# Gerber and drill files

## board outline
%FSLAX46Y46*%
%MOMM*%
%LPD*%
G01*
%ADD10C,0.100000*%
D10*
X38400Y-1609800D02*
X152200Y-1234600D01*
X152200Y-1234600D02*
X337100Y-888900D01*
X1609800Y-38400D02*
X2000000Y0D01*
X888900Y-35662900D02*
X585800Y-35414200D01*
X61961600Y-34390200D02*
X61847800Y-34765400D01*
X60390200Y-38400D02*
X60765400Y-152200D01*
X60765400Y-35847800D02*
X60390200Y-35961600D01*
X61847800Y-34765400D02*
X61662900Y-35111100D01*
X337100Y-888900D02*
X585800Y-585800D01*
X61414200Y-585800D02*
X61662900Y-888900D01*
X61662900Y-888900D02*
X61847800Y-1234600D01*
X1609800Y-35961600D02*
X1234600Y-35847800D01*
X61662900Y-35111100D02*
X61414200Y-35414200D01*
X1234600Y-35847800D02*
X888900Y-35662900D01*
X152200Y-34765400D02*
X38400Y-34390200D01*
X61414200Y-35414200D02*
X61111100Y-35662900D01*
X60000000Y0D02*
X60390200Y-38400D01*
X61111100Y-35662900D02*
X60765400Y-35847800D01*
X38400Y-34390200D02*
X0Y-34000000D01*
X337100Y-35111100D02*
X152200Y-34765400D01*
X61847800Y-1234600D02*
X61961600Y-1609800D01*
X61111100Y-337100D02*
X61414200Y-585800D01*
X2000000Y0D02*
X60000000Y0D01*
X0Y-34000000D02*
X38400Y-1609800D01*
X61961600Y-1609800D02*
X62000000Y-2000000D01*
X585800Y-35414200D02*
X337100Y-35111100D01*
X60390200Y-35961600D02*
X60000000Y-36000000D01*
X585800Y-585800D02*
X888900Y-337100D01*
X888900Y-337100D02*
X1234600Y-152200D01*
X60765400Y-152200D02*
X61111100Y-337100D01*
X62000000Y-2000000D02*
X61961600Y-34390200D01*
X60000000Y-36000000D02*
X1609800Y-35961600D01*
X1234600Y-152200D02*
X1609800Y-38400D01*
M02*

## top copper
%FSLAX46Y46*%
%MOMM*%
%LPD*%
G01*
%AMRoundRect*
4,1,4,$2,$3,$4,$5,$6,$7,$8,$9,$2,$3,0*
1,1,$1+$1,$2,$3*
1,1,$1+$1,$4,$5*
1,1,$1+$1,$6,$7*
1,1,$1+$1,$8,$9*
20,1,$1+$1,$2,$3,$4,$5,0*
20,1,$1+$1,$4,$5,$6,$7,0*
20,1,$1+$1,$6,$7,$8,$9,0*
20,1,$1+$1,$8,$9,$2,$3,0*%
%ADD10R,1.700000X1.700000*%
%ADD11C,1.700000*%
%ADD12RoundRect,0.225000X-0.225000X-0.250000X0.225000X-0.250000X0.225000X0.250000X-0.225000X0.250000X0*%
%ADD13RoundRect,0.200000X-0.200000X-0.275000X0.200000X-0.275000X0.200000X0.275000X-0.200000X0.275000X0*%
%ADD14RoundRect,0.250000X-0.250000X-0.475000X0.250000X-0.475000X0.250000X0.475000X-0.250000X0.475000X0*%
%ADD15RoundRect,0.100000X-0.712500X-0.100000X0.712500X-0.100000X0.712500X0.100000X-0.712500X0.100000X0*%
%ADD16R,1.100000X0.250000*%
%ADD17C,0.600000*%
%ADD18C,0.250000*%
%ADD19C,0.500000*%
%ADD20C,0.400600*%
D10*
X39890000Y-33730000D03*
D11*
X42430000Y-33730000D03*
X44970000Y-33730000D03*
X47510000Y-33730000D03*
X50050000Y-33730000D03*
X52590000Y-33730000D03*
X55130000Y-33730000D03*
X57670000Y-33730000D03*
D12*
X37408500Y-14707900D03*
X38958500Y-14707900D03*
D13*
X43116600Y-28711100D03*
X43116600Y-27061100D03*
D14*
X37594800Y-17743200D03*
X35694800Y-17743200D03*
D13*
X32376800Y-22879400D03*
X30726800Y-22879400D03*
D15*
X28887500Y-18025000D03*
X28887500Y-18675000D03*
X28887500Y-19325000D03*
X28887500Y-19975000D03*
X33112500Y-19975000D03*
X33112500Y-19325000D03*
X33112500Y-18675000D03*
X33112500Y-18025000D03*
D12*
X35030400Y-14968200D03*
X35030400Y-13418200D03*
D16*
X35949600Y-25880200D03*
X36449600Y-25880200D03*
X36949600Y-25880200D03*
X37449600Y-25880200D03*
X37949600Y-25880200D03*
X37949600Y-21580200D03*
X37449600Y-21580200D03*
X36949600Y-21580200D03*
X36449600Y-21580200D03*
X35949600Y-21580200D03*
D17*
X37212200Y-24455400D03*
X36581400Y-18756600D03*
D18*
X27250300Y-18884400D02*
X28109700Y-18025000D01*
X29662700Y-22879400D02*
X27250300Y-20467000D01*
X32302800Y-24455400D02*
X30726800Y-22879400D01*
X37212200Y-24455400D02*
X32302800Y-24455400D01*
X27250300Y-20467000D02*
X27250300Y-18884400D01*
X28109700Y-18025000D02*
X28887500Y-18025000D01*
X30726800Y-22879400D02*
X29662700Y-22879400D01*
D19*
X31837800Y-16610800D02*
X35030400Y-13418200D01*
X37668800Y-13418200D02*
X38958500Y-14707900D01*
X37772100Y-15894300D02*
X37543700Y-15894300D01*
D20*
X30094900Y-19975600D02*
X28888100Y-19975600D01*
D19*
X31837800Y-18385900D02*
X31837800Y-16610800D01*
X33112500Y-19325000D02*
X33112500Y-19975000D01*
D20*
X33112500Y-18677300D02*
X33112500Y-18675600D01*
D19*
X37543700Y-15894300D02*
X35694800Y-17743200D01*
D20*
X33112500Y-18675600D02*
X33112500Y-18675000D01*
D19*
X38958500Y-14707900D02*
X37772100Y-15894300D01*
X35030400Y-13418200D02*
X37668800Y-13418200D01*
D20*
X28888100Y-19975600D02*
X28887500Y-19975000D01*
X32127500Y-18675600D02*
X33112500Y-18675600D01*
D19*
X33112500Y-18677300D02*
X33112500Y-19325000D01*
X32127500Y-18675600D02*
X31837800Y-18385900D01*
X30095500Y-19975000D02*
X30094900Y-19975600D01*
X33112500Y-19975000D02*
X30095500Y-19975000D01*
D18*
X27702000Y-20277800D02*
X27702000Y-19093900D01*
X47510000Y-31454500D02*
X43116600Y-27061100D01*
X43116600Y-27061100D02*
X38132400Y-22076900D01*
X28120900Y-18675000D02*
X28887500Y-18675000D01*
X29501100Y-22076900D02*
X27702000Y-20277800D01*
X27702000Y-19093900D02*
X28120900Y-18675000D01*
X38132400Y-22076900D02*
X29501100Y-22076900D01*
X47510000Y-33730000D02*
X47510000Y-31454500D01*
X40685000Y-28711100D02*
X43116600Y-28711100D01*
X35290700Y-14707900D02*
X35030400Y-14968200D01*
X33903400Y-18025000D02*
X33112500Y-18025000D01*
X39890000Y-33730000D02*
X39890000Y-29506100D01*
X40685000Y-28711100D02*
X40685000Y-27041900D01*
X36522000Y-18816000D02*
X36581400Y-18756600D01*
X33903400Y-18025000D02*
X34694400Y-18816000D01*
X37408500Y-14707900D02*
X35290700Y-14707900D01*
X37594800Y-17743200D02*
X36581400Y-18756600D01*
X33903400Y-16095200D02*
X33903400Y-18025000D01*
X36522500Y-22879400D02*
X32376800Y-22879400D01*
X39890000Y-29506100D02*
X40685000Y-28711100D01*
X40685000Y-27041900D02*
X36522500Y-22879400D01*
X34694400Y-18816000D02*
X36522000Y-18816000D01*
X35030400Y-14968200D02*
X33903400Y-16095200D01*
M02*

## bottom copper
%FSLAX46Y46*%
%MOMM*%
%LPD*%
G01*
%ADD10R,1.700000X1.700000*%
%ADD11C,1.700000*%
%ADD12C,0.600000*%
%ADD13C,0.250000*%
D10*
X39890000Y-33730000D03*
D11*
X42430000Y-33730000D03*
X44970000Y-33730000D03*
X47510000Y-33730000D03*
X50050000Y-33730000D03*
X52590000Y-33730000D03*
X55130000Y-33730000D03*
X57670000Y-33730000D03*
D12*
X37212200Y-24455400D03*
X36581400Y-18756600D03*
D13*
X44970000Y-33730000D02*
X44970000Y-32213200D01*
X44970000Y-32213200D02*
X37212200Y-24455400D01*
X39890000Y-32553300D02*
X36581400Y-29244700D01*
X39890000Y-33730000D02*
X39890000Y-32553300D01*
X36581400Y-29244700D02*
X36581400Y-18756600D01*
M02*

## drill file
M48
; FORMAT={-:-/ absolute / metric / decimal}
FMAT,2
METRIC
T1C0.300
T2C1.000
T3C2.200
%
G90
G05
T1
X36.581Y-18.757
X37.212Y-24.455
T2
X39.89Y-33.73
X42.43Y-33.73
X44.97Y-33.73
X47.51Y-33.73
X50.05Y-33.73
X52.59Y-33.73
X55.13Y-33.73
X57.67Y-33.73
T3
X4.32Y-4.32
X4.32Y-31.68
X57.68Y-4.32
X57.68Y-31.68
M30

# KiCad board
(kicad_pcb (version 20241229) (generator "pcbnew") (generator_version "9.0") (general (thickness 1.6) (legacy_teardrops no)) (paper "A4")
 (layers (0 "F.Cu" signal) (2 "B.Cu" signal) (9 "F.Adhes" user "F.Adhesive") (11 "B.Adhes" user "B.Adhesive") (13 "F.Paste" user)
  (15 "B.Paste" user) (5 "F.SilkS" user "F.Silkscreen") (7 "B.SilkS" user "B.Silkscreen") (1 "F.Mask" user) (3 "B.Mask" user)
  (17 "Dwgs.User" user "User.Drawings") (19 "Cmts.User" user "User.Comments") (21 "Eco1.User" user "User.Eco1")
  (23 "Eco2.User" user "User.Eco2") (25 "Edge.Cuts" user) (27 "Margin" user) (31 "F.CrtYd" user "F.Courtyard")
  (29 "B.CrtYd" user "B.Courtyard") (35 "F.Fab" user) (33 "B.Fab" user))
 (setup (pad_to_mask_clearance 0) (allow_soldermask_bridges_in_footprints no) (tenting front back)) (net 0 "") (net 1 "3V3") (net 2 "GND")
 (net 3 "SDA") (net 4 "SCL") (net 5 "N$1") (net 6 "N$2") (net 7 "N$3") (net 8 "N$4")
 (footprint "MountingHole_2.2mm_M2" (layer "F.Cu") (at 4.32 4.32)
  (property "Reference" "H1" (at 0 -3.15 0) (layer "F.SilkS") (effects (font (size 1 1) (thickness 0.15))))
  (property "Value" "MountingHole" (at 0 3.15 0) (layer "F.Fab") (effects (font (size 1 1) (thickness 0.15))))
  (pad "" np_thru_hole circle (at 0 0) (size 2.2 2.2) (drill 2.2) (layers "*.Cu" "*.Mask")))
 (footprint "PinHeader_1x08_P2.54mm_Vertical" (layer "F.Cu") (at 39.89 33.73 90)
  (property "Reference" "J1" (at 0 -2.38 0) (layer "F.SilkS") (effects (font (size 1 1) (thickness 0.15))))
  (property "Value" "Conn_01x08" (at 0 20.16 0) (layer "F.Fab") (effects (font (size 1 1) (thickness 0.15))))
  (pad "1" thru_hole rect (at 0 0) (size 1.7 1.7) (drill 1) (layers "*.Cu" "*.Mask") (remove_unused_layers no) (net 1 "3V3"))
  (pad "2" thru_hole circle (at 0 2.54) (size 1.7 1.7) (drill 1) (layers "*.Cu" "*.Mask") (remove_unused_layers no) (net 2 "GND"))
  (pad "3" thru_hole circle (at 0 5.08) (size 1.7 1.7) (drill 1) (layers "*.Cu" "*.Mask") (remove_unused_layers no) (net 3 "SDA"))
  (pad "4" thru_hole circle (at 0 7.62) (size 1.7 1.7) (drill 1) (layers "*.Cu" "*.Mask") (remove_unused_layers no) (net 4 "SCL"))
  (pad "5" thru_hole circle (at 0 10.16) (size 1.7 1.7) (drill 1) (layers "*.Cu" "*.Mask") (remove_unused_layers no) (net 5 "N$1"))
  (pad "6" thru_hole circle (at 0 12.7) (size 1.7 1.7) (drill 1) (layers "*.Cu" "*.Mask") (remove_unused_layers no) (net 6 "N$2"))
  (pad "7" thru_hole circle (at 0 15.24) (size 1.7 1.7) (drill 1) (layers "*.Cu" "*.Mask") (remove_unused_layers no) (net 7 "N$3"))
  (pad "8" thru_hole circle (at 0 17.78) (size 1.7 1.7) (drill 1) (layers "*.Cu" "*.Mask") (remove_unused_layers no) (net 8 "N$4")))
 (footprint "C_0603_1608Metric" (layer "F.Cu") (at 38.1835 14.7079)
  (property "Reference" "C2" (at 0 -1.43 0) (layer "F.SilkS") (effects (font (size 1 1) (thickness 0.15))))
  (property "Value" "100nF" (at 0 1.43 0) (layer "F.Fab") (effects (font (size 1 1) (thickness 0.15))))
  (pad "1" smd roundrect (at -0.775 0) (size 0.9 0.95) (layers "F.Cu" "F.Mask" "F.Paste") (roundrect_rratio 0.25) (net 1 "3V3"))
  (pad "2" smd roundrect (at 0.775 0) (size 0.9 0.95) (layers "F.Cu" "F.Mask" "F.Paste") (roundrect_rratio 0.25) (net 2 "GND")))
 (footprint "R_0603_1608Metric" (layer "F.Cu") (at 43.1166 27.8861 90)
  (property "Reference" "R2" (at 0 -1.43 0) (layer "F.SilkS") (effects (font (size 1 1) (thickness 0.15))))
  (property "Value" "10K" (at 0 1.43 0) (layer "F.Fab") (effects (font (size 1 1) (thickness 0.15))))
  (pad "1" smd roundrect (at -0.825 0) (size 0.8 0.95) (layers "F.Cu" "F.Mask" "F.Paste") (roundrect_rratio 0.25) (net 1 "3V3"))
  (pad "2" smd roundrect (at 0.825 0) (size 0.8 0.95) (layers "F.Cu" "F.Mask" "F.Paste") (roundrect_rratio 0.25) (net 4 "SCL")))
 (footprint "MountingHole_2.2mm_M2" (layer "F.Cu") (at 57.68 31.68)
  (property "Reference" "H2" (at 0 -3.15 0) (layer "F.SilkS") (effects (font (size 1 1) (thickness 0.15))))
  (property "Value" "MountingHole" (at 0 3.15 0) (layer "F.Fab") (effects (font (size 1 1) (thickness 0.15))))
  (pad "" np_thru_hole circle (at 0 0) (size 2.2 2.2) (drill 2.2) (layers "*.Cu" "*.Mask")))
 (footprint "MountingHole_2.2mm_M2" (layer "F.Cu") (at 4.32 31.68)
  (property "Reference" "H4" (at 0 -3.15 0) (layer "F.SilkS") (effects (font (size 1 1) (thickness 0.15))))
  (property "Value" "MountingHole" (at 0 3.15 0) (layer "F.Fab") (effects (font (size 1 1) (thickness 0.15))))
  (pad "" np_thru_hole circle (at 0 0) (size 2.2 2.2) (drill 2.2) (layers "*.Cu" "*.Mask")))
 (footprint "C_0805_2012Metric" (layer "F.Cu") (at 36.6448 17.7432 180)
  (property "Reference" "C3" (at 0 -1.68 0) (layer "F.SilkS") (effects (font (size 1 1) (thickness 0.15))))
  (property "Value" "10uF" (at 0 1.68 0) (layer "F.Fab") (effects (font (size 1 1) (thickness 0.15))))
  (pad "1" smd roundrect (at -0.95 0) (size 1 1.45) (layers "F.Cu" "F.Mask" "F.Paste") (roundrect_rratio 0.25) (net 1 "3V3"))
  (pad "2" smd roundrect (at 0.95 0) (size 1 1.45) (layers "F.Cu" "F.Mask" "F.Paste") (roundrect_rratio 0.25) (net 2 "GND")))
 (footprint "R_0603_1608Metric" (layer "F.Cu") (at 31.5518 22.8794 180)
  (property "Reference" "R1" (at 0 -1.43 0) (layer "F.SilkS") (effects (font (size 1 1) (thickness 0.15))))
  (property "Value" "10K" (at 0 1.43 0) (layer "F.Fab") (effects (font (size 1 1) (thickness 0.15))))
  (pad "1" smd roundrect (at -0.825 0) (size 0.8 0.95) (layers "F.Cu" "F.Mask" "F.Paste") (roundrect_rratio 0.25) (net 1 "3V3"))
  (pad "2" smd roundrect (at 0.825 0) (size 0.8 0.95) (layers "F.Cu" "F.Mask" "F.Paste") (roundrect_rratio 0.25) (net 3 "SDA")))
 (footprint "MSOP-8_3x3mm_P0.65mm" (layer "F.Cu") (at 31 19)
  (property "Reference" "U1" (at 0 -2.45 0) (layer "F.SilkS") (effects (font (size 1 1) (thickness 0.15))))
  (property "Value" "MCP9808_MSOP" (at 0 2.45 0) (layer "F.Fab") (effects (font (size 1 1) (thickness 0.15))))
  (pad "1" smd roundrect (at -2.1125 -0.975) (size 1.625 0.4) (layers "F.Cu" "F.Mask" "F.Paste") (roundrect_rratio 0.25) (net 3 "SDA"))
  (pad "2" smd roundrect (at -2.1125 -0.325) (size 1.625 0.4) (layers "F.Cu" "F.Mask" "F.Paste") (roundrect_rratio 0.25) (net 4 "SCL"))
  (pad "3" smd roundrect (at -2.1125 0.325) (size 1.625 0.4) (layers "F.Cu" "F.Mask" "F.Paste") (roundrect_rratio 0.25))
  (pad "4" smd roundrect (at -2.1125 0.975) (size 1.625 0.4) (layers "F.Cu" "F.Mask" "F.Paste") (roundrect_rratio 0.25) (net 2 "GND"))
  (pad "5" smd roundrect (at 2.1125 0.975) (size 1.625 0.4) (layers "F.Cu" "F.Mask" "F.Paste") (roundrect_rratio 0.25) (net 2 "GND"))
  (pad "6" smd roundrect (at 2.1125 0.325) (size 1.625 0.4) (layers "F.Cu" "F.Mask" "F.Paste") (roundrect_rratio 0.25) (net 2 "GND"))
  (pad "7" smd roundrect (at 2.1125 -0.325) (size 1.625 0.4) (layers "F.Cu" "F.Mask" "F.Paste") (roundrect_rratio 0.25) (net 2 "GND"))
  (pad "8" smd roundrect (at 2.1125 -0.975) (size 1.625 0.4) (layers "F.Cu" "F.Mask" "F.Paste") (roundrect_rratio 0.25) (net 1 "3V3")))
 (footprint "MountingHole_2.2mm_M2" (layer "F.Cu") (at 57.68 4.32)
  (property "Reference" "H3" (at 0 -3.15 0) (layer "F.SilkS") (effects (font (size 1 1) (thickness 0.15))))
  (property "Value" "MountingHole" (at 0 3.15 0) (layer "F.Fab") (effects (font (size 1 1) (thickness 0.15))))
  (pad "" np_thru_hole circle (at 0 0) (size 2.2 2.2) (drill 2.2) (layers "*.Cu" "*.Mask")))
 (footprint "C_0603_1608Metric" (layer "F.Cu") (at 35.0304 14.1932 90)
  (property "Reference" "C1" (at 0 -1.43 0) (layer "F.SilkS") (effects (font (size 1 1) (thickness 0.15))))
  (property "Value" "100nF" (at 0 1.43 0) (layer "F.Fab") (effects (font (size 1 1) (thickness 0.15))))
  (pad "1" smd roundrect (at -0.775 0) (size 0.9 0.95) (layers "F.Cu" "F.Mask" "F.Paste") (roundrect_rratio 0.25) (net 1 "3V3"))
  (pad "2" smd roundrect (at 0.775 0) (size 0.9 0.95) (layers "F.Cu" "F.Mask" "F.Paste") (roundrect_rratio 0.25) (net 2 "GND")))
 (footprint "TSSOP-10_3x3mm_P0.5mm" (layer "F.Cu") (at 36.9496 23.7302 90)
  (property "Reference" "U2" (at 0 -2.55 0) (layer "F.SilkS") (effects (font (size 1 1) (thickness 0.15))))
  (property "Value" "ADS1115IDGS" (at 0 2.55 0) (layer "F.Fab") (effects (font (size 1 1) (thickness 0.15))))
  (pad "1" smd rect (at -2.15 -1) (size 1.1 0.25) (layers "F.Cu" "F.Mask" "F.Paste") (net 2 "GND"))
  (pad "2" smd rect (at -2.15 -0.5) (size 1.1 0.25) (layers "F.Cu" "F.Mask" "F.Paste"))
  (pad "3" smd rect (at -2.15 0) (size 1.1 0.25) (layers "F.Cu" "F.Mask" "F.Paste") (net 2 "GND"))
  (pad "4" smd rect (at -2.15 0.5) (size 1.1 0.25) (layers "F.Cu" "F.Mask" "F.Paste") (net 5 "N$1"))
  (pad "5" smd rect (at -2.15 1) (size 1.1 0.25) (layers "F.Cu" "F.Mask" "F.Paste") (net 6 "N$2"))
  (pad "6" smd rect (at 2.15 1) (size 1.1 0.25) (layers "F.Cu" "F.Mask" "F.Paste") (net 7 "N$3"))
  (pad "7" smd rect (at 2.15 0.5) (size 1.1 0.25) (layers "F.Cu" "F.Mask" "F.Paste") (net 8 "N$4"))
  (pad "8" smd rect (at 2.15 0) (size 1.1 0.25) (layers "F.Cu" "F.Mask" "F.Paste") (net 1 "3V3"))
  (pad "9" smd rect (at 2.15 -0.5) (size 1.1 0.25) (layers "F.Cu" "F.Mask" "F.Paste") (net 3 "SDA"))
  (pad "10" smd rect (at 2.15 -1) (size 1.1 0.25) (layers "F.Cu" "F.Mask" "F.Paste") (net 4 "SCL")))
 (gr_line (start 0.0384 1.6098) (end 0.1522 1.2346) (stroke (width 0.1) (type solid)) (layer "Edge.Cuts"))
 (gr_line (start 0.1522 1.2346) (end 0.3371 0.8889) (stroke (width 0.1) (type solid)) (layer "Edge.Cuts"))
 (gr_line (start 1.6098 0.0384) (end 2 0) (stroke (width 0.1) (type solid)) (layer "Edge.Cuts"))
 (gr_line (start 0.8889 35.6629) (end 0.5858 35.4142) (stroke (width 0.1) (type solid)) (layer "Edge.Cuts"))
 (gr_line (start 61.9616 34.3902) (end 61.8478 34.7654) (stroke (width 0.1) (type solid)) (layer "Edge.Cuts"))
 (gr_line (start 60.3902 0.0384) (end 60.7654 0.1522) (stroke (width 0.1) (type solid)) (layer "Edge.Cuts"))
 (gr_line (start 60.7654 35.8478) (end 60.3902 35.9616) (stroke (width 0.1) (type solid)) (layer "Edge.Cuts"))
 (gr_line (start 61.8478 34.7654) (end 61.6629 35.1111) (stroke (width 0.1) (type solid)) (layer "Edge.Cuts"))
 (gr_line (start 0.3371 0.8889) (end 0.5858 0.5858) (stroke (width 0.1) (type solid)) (layer "Edge.Cuts"))
 (gr_line (start 61.4142 0.5858) (end 61.6629 0.8889) (stroke (width 0.1) (type solid)) (layer "Edge.Cuts"))
 (gr_line (start 61.6629 0.8889) (end 61.8478 1.2346) (stroke (width 0.1) (type solid)) (layer "Edge.Cuts"))
 (gr_line (start 1.6098 35.9616) (end 1.2346 35.8478) (stroke (width 0.1) (type solid)) (layer "Edge.Cuts"))
 (gr_line (start 61.6629 35.1111) (end 61.4142 35.4142) (stroke (width 0.1) (type solid)) (layer "Edge.Cuts"))
 (gr_line (start 1.2346 35.8478) (end 0.8889 35.6629) (stroke (width 0.1) (type solid)) (layer "Edge.Cuts"))
 (gr_line (start 0.1522 34.7654) (end 0.0384 34.3902) (stroke (width 0.1) (type solid)) (layer "Edge.Cuts"))
 (gr_line (start 61.4142 35.4142) (end 61.1111 35.6629) (stroke (width 0.1) (type solid)) (layer "Edge.Cuts"))
 (gr_line (start 60 0) (end 60.3902 0.0384) (stroke (width 0.1) (type solid)) (layer "Edge.Cuts"))
 (gr_line (start 61.1111 35.6629) (end 60.7654 35.8478) (stroke (width 0.1) (type solid)) (layer "Edge.Cuts"))
 (gr_line (start 0.0384 34.3902) (end 0 34) (stroke (width 0.1) (type solid)) (layer "Edge.Cuts"))
 (gr_line (start 0.3371 35.1111) (end 0.1522 34.7654) (stroke (width 0.1) (type solid)) (layer "Edge.Cuts"))
 (gr_line (start 61.8478 1.2346) (end 61.9616 1.6098) (stroke (width 0.1) (type solid)) (layer "Edge.Cuts"))
 (gr_line (start 61.1111 0.3371) (end 61.4142 0.5858) (stroke (width 0.1) (type solid)) (layer "Edge.Cuts"))
 (gr_line (start 2 0) (end 60 0) (stroke (width 0.1) (type solid)) (layer "Edge.Cuts"))
 (gr_line (start 0 34) (end 0.0384 1.6098) (stroke (width 0.1) (type solid)) (layer "Edge.Cuts"))
 (gr_line (start 61.9616 1.6098) (end 62 2) (stroke (width 0.1) (type solid)) (layer "Edge.Cuts"))
 (gr_line (start 0.5858 35.4142) (end 0.3371 35.1111) (stroke (width 0.1) (type solid)) (layer "Edge.Cuts"))
 (gr_line (start 60.3902 35.9616) (end 60 36) (stroke (width 0.1) (type solid)) (layer "Edge.Cuts"))
 (gr_line (start 0.5858 0.5858) (end 0.8889 0.3371) (stroke (width 0.1) (type solid)) (layer "Edge.Cuts"))
 (gr_line (start 0.8889 0.3371) (end 1.2346 0.1522) (stroke (width 0.1) (type solid)) (layer "Edge.Cuts"))
 (gr_line (start 60.7654 0.1522) (end 61.1111 0.3371) (stroke (width 0.1) (type solid)) (layer "Edge.Cuts"))
 (gr_line (start 62 2) (end 61.9616 34.3902) (stroke (width 0.1) (type solid)) (layer "Edge.Cuts"))
 (gr_line (start 60 36) (end 1.6098 35.9616) (stroke (width 0.1) (type solid)) (layer "Edge.Cuts"))
 (gr_line (start 1.2346 0.1522) (end 1.6098 0.0384) (stroke (width 0.1) (type solid)) (layer "Edge.Cuts"))
 (segment (start 27.2503 18.8844) (end 28.1097 18.025) (width 0.25) (layer "F.Cu") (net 3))
 (segment (start 29.6627 22.8794) (end 27.2503 20.467) (width 0.25) (layer "F.Cu") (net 3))
 (segment (start 32.3028 24.4554) (end 30.7268 22.8794) (width 0.25) (layer "F.Cu") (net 3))
 (segment (start 37.2122 24.4554) (end 32.3028 24.4554) (width 0.25) (layer "F.Cu") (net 3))
 (segment (start 27.2503 20.467) (end 27.2503 18.8844) (width 0.25) (layer "F.Cu") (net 3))
 (segment (start 28.1097 18.025) (end 28.8875 18.025) (width 0.25) (layer "F.Cu") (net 3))
 (segment (start 30.7268 22.8794) (end 29.6627 22.8794) (width 0.25) (layer "F.Cu") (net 3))
 (via (at 37.2122 24.4554) (size 0.6) (drill 0.3) (layers "F.Cu" "B.Cu") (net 3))
 (segment (start 44.97 33.73) (end 44.97 32.2132) (width 0.25) (layer "B.Cu") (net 3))
 (segment (start 44.97 32.2132) (end 37.2122 24.4554) (width 0.25) (layer "B.Cu") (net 3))
 (segment (start 31.8378 16.6108) (end 35.0304 13.4182) (width 0.5) (layer "F.Cu") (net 2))
 (segment (start 37.6688 13.4182) (end 38.9585 14.7079) (width 0.5) (layer "F.Cu") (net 2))
 (segment (start 37.7721 15.8943) (end 37.5437 15.8943) (width 0.5) (layer "F.Cu") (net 2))
 (segment (start 30.0949 19.9756) (end 28.8881 19.9756) (width 0.4006) (layer "F.Cu") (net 2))
 (segment (start 31.8378 18.3859) (end 31.8378 16.6108) (width 0.5) (layer "F.Cu") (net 2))
 (segment (start 33.1125 19.325) (end 33.1125 19.975) (width 0.5) (layer "F.Cu") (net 2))
 (segment (start 33.1125 18.6773) (end 33.1125 18.6756) (width 0.4006) (layer "F.Cu") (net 2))
 (segment (start 37.5437 15.8943) (end 35.6948 17.7432) (width 0.5) (layer "F.Cu") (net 2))
 (segment (start 33.1125 18.6756) (end 33.1125 18.675) (width 0.4006) (layer "F.Cu") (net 2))
 (segment (start 38.9585 14.7079) (end 37.7721 15.8943) (width 0.5) (layer "F.Cu") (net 2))
 (segment (start 35.0304 13.4182) (end 37.6688 13.4182) (width 0.5) (layer "F.Cu") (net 2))
 (segment (start 28.8881 19.9756) (end 28.8875 19.975) (width 0.4006) (layer "F.Cu") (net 2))
 (segment (start 32.1275 18.6756) (end 33.1125 18.6756) (width 0.4006) (layer "F.Cu") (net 2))
 (segment (start 33.1125 18.6773) (end 33.1125 19.325) (width 0.5) (layer "F.Cu") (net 2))
 (segment (start 32.1275 18.6756) (end 31.8378 18.3859) (width 0.5) (layer "F.Cu") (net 2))
 (segment (start 30.0955 19.975) (end 30.0949 19.9756) (width 0.5) (layer "F.Cu") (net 2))
 (segment (start 33.1125 19.975) (end 30.0955 19.975) (width 0.5) (layer "F.Cu") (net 2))
 (segment (start 27.702 20.2778) (end 27.702 19.0939) (width 0.25) (layer "F.Cu") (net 4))
 (segment (start 47.51 31.4545) (end 43.1166 27.0611) (width 0.25) (layer "F.Cu") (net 4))
 (segment (start 43.1166 27.0611) (end 38.1324 22.0769) (width 0.25) (layer "F.Cu") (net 4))
 (segment (start 28.1209 18.675) (end 28.8875 18.675) (width 0.25) (layer "F.Cu") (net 4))
 (segment (start 29.5011 22.0769) (end 27.702 20.2778) (width 0.25) (layer "F.Cu") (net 4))
 (segment (start 27.702 19.0939) (end 28.1209 18.675) (width 0.25) (layer "F.Cu") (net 4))
 (segment (start 38.1324 22.0769) (end 29.5011 22.0769) (width 0.25) (layer "F.Cu") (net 4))
 (segment (start 47.51 33.73) (end 47.51 31.4545) (width 0.25) (layer "F.Cu") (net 4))
 (segment (start 40.685 28.7111) (end 43.1166 28.7111) (width 0.25) (layer "F.Cu") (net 1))
 (segment (start 35.2907 14.7079) (end 35.0304 14.9682) (width 0.25) (layer "F.Cu") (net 1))
 (segment (start 33.9034 18.025) (end 33.1125 18.025) (width 0.25) (layer "F.Cu") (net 1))
 (segment (start 39.89 33.73) (end 39.89 29.5061) (width 0.25) (layer "F.Cu") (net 1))
 (segment (start 40.685 28.7111) (end 40.685 27.0419) (width 0.25) (layer "F.Cu") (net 1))
 (segment (start 36.522 18.816) (end 36.5814 18.7566) (width 0.25) (layer "F.Cu") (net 1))
 (segment (start 33.9034 18.025) (end 34.6944 18.816) (width 0.25) (layer "F.Cu") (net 1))
 (segment (start 37.4085 14.7079) (end 35.2907 14.7079) (width 0.25) (layer "F.Cu") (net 1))
 (segment (start 37.5948 17.7432) (end 36.5814 18.7566) (width 0.25) (layer "F.Cu") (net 1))
 (segment (start 33.9034 16.0952) (end 33.9034 18.025) (width 0.25) (layer "F.Cu") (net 1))
 (segment (start 36.5225 22.8794) (end 32.3768 22.8794) (width 0.25) (layer "F.Cu") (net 1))
 (segment (start 39.89 29.5061) (end 40.685 28.7111) (width 0.25) (layer "F.Cu") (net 1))
 (segment (start 40.685 27.0419) (end 36.5225 22.8794) (width 0.25) (layer "F.Cu") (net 1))
 (segment (start 34.6944 18.816) (end 36.522 18.816) (width 0.25) (layer "F.Cu") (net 1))
 (segment (start 35.0304 14.9682) (end 33.9034 16.0952) (width 0.25) (layer "F.Cu") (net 1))
 (via (at 36.5814 18.7566) (size 0.6) (drill 0.3) (layers "F.Cu" "B.Cu") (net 1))
 (segment (start 39.89 32.5533) (end 36.5814 29.2447) (width 0.25) (layer "B.Cu") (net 1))
 (segment (start 39.89 33.73) (end 39.89 32.5533) (width 0.25) (layer "B.Cu") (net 1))
 (segment (start 36.5814 29.2447) (end 36.5814 18.7566) (width 0.25) (layer "B.Cu") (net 1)))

